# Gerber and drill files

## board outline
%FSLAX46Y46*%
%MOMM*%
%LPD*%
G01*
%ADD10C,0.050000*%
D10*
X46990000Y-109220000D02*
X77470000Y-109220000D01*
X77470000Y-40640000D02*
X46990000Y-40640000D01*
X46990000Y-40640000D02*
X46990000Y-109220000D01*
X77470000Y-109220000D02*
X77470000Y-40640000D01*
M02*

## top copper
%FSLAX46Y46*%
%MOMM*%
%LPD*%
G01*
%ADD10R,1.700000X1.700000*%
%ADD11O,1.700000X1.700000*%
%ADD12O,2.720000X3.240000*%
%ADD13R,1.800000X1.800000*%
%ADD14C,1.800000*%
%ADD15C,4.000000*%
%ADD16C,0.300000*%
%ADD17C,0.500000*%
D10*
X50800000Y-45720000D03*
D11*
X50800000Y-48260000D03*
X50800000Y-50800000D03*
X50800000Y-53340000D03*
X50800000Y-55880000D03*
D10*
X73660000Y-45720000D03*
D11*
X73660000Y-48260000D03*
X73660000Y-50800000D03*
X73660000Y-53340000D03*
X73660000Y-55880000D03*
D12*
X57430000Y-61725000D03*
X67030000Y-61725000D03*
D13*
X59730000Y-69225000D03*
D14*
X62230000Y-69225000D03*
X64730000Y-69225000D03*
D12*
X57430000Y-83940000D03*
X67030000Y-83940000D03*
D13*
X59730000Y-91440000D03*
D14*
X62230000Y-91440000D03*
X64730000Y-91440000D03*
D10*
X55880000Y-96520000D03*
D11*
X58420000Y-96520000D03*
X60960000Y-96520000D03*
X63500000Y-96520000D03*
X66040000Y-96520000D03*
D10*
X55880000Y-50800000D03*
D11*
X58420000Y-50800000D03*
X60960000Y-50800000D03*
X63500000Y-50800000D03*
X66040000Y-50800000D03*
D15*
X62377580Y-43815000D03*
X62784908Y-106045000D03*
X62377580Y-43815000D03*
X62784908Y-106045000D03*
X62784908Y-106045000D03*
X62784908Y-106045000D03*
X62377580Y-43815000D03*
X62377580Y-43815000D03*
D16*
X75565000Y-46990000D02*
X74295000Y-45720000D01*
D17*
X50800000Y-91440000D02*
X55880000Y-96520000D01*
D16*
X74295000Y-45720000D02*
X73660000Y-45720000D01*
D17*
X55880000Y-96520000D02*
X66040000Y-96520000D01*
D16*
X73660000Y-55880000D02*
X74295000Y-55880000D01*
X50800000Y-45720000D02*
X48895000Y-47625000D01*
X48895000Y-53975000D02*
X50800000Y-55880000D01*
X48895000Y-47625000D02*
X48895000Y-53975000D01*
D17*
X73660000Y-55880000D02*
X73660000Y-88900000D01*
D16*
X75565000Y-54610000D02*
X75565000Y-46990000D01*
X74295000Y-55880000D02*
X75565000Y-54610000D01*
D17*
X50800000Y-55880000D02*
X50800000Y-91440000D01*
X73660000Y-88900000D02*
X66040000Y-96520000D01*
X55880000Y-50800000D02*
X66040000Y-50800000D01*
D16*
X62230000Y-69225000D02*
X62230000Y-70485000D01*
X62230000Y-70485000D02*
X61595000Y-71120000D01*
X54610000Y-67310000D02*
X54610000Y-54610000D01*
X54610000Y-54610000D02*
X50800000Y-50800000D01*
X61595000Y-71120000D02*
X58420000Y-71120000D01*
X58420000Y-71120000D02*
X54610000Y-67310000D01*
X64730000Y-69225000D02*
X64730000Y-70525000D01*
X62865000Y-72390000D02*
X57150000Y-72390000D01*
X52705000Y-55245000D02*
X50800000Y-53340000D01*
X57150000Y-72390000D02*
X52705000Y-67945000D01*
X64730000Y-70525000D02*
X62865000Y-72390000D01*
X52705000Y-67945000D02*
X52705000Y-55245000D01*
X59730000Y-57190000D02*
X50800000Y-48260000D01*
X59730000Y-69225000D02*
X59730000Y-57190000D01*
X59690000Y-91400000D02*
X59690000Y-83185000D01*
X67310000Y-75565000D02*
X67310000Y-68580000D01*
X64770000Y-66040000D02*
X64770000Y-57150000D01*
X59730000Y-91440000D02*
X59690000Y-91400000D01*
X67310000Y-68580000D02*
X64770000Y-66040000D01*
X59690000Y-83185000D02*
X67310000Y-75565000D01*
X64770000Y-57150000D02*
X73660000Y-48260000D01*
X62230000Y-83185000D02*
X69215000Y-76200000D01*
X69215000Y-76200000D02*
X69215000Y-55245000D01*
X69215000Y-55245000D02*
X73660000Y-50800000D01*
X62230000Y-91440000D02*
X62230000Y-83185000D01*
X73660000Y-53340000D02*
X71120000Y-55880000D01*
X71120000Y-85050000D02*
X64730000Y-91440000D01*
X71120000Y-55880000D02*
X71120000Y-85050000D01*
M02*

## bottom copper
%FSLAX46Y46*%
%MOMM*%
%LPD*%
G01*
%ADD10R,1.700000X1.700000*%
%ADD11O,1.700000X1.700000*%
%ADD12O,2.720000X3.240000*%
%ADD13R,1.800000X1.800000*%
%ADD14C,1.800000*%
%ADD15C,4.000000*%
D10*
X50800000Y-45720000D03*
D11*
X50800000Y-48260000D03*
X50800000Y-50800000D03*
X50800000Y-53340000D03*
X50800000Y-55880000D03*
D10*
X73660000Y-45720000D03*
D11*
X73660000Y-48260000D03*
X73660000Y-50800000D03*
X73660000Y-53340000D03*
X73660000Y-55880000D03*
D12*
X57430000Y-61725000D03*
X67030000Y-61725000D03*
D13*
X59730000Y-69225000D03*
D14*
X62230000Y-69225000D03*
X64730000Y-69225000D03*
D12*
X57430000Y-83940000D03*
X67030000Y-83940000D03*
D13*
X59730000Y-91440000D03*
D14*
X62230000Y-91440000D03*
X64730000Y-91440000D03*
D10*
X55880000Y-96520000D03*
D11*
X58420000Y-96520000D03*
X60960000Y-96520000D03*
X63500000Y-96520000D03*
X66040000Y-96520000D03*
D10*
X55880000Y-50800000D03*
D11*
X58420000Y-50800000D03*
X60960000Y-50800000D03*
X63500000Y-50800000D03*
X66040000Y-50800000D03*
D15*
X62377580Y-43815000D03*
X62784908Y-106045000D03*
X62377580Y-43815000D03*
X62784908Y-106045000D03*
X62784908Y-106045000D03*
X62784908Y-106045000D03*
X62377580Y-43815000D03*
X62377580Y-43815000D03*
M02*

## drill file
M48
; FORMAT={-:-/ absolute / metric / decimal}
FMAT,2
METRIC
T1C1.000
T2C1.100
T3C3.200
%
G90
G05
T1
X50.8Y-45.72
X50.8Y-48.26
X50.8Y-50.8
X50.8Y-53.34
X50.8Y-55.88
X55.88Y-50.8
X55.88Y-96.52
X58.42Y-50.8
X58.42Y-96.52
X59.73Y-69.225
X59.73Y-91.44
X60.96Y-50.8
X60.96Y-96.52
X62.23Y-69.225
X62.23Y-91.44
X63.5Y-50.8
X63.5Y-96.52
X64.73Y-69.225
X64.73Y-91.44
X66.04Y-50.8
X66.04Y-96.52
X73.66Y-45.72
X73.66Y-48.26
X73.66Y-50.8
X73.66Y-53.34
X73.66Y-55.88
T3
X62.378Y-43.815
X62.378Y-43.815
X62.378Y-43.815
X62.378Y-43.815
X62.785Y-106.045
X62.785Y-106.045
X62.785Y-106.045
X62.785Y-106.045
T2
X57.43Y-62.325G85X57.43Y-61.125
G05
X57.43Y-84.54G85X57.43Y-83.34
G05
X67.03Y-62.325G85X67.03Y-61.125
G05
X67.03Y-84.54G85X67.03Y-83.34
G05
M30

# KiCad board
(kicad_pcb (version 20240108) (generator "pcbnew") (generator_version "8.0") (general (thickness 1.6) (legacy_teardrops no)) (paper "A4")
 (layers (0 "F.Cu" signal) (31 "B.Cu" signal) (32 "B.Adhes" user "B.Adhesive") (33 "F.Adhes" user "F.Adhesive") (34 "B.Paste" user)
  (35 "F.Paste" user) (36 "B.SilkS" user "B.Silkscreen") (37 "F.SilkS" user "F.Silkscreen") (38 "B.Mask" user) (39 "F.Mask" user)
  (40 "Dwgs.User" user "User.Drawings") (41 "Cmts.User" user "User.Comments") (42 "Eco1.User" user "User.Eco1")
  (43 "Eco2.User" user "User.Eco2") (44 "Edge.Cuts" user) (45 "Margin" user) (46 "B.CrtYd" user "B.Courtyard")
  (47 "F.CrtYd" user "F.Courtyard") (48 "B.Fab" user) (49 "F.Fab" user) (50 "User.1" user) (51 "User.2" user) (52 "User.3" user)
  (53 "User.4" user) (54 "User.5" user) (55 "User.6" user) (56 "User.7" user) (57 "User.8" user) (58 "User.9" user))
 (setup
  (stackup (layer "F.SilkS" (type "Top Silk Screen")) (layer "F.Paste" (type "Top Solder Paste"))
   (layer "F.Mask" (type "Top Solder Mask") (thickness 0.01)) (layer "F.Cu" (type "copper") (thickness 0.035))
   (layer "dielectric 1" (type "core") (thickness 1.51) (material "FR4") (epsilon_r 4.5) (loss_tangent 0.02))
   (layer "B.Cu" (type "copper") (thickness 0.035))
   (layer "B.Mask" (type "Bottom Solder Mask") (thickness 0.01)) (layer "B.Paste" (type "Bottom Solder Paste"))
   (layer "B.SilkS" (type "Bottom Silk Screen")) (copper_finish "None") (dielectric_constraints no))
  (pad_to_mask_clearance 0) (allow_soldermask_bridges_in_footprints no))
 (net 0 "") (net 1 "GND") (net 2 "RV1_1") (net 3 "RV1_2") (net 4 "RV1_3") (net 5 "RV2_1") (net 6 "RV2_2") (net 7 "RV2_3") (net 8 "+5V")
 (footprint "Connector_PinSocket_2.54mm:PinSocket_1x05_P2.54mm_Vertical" (layer "F.Cu") (at 50.8 45.72)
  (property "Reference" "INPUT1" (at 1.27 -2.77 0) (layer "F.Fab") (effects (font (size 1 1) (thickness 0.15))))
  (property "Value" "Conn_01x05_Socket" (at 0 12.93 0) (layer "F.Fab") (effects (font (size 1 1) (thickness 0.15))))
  (pad "1" thru_hole rect (at 0 0) (size 1.7 1.7) (drill 1) (layers "*.Cu" "*.Mask") (remove_unused_layers no) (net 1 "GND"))
  (pad "2" thru_hole oval (at 0 2.54) (size 1.7 1.7) (drill 1) (layers "*.Cu" "*.Mask") (remove_unused_layers no) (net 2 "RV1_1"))
  (pad "3" thru_hole oval (at 0 5.08) (size 1.7 1.7) (drill 1) (layers "*.Cu" "*.Mask") (remove_unused_layers no) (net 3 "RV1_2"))
  (pad "4" thru_hole oval (at 0 7.62) (size 1.7 1.7) (drill 1) (layers "*.Cu" "*.Mask") (remove_unused_layers no) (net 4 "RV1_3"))
  (pad "5" thru_hole oval (at 0 10.16) (size 1.7 1.7) (drill 1) (layers "*.Cu" "*.Mask") (remove_unused_layers no) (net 1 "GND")))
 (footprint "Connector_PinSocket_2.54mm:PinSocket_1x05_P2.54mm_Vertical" (layer "F.Cu") (at 73.66 45.72)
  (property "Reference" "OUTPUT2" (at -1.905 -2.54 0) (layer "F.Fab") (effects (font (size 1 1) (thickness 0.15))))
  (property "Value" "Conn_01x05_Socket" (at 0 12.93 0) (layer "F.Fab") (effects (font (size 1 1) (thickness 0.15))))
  (pad "1" thru_hole rect (at 0 0) (size 1.7 1.7) (drill 1) (layers "*.Cu" "*.Mask") (remove_unused_layers no) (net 1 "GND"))
  (pad "2" thru_hole oval (at 0 2.54) (size 1.7 1.7) (drill 1) (layers "*.Cu" "*.Mask") (remove_unused_layers no) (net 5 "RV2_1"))
  (pad "3" thru_hole oval (at 0 5.08) (size 1.7 1.7) (drill 1) (layers "*.Cu" "*.Mask") (remove_unused_layers no) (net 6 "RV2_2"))
  (pad "4" thru_hole oval (at 0 7.62) (size 1.7 1.7) (drill 1) (layers "*.Cu" "*.Mask") (remove_unused_layers no) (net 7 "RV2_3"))
  (pad "5" thru_hole oval (at 0 10.16) (size 1.7 1.7) (drill 1) (layers "*.Cu" "*.Mask") (remove_unused_layers no) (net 1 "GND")))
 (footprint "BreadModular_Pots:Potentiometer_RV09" (layer "F.Cu") (at 59.73 69.225 90)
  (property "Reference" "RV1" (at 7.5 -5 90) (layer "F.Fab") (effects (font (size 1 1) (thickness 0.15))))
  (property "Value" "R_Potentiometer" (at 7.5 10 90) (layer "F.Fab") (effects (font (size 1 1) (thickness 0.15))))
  (pad "" thru_hole oval (at 7.5 -2.3 180) (size 2.72 3.24) (drill oval 1.1 2.3) (layers "*.Cu" "*.Mask") (remove_unused_layers no))
  (pad "" thru_hole oval (at 7.5 7.3 180) (size 2.72 3.24) (drill oval 1.1 2.3) (layers "*.Cu" "*.Mask") (remove_unused_layers no))
  (pad "1" thru_hole rect (at 0 0 180) (size 1.8 1.8) (drill 1) (layers "*.Cu" "*.Mask") (remove_unused_layers no) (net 2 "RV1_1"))
  (pad "2" thru_hole circle (at 0 2.5 180) (size 1.8 1.8) (drill 1) (layers "*.Cu" "*.Mask") (remove_unused_layers no) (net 3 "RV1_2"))
  (pad "3" thru_hole circle (at 0 5 180) (size 1.8 1.8) (drill 1) (layers "*.Cu" "*.Mask") (remove_unused_layers no) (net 4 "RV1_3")))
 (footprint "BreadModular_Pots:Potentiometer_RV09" (layer "F.Cu") (at 59.73 91.44 90)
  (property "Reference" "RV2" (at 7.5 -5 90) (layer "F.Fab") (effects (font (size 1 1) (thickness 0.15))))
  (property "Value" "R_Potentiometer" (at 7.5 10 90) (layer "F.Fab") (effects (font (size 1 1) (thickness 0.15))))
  (pad "" thru_hole oval (at 7.5 -2.3 180) (size 2.72 3.24) (drill oval 1.1 2.3) (layers "*.Cu" "*.Mask") (remove_unused_layers no))
  (pad "" thru_hole oval (at 7.5 7.3 180) (size 2.72 3.24) (drill oval 1.1 2.3) (layers "*.Cu" "*.Mask") (remove_unused_layers no))
  (pad "1" thru_hole rect (at 0 0 180) (size 1.8 1.8) (drill 1) (layers "*.Cu" "*.Mask") (remove_unused_layers no) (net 5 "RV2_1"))
  (pad "2" thru_hole circle (at 0 2.5 180) (size 1.8 1.8) (drill 1) (layers "*.Cu" "*.Mask") (remove_unused_layers no) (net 6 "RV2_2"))
  (pad "3" thru_hole circle (at 0 5 180) (size 1.8 1.8) (drill 1) (layers "*.Cu" "*.Mask") (remove_unused_layers no) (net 7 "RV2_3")))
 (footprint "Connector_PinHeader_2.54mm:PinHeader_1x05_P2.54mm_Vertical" (layer "B.Cu") (at 55.88 96.52 -90)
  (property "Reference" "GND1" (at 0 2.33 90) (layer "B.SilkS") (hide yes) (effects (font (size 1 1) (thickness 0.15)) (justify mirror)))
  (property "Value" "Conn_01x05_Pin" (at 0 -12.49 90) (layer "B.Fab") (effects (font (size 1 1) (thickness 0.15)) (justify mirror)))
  (pad "1" thru_hole rect (at 0 0 270) (size 1.7 1.7) (drill 1) (layers "*.Cu" "*.Mask") (remove_unused_layers no) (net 1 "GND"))
  (pad "2" thru_hole oval (at 0 -2.54 270) (size 1.7 1.7) (drill 1) (layers "*.Cu" "*.Mask") (remove_unused_layers no) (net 1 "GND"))
  (pad "3" thru_hole oval (at 0 -5.08 270) (size 1.7 1.7) (drill 1) (layers "*.Cu" "*.Mask") (remove_unused_layers no) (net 1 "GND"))
  (pad "4" thru_hole oval (at 0 -7.62 270) (size 1.7 1.7) (drill 1) (layers "*.Cu" "*.Mask") (remove_unused_layers no) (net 1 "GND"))
  (pad "5" thru_hole oval (at 0 -10.16 270) (size 1.7 1.7) (drill 1) (layers "*.Cu" "*.Mask") (remove_unused_layers no) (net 1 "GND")))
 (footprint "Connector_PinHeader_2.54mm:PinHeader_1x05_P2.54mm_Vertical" (layer "B.Cu") (at 55.88 50.8 -90)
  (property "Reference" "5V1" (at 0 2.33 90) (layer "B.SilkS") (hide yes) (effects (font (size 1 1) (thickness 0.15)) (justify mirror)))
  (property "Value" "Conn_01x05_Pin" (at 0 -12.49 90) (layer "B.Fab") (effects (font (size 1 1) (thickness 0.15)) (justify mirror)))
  (pad "1" thru_hole rect (at 0 0 270) (size 1.7 1.7) (drill 1) (layers "*.Cu" "*.Mask") (remove_unused_layers no) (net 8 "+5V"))
  (pad "2" thru_hole oval (at 0 -2.54 270) (size 1.7 1.7) (drill 1) (layers "*.Cu" "*.Mask") (remove_unused_layers no) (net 8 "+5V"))
  (pad "3" thru_hole oval (at 0 -5.08 270) (size 1.7 1.7) (drill 1) (layers "*.Cu" "*.Mask") (remove_unused_layers no) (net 8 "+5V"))
  (pad "4" thru_hole oval (at 0 -7.62 270) (size 1.7 1.7) (drill 1) (layers "*.Cu" "*.Mask") (remove_unused_layers no) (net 8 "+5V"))
  (pad "5" thru_hole oval (at 0 -10.16 270) (size 1.7 1.7) (drill 1) (layers "*.Cu" "*.Mask") (remove_unused_layers no) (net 8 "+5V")))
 (gr_line (start 46.99 109.22) (end 77.47 109.22) (stroke (width 0.05) (type default)) (layer "Edge.Cuts"))
 (gr_line (start 77.47 40.64) (end 46.99 40.64) (stroke (width 0.05) (type default)) (layer "Edge.Cuts"))
 (gr_line (start 46.99 40.64) (end 46.99 109.22) (stroke (width 0.05) (type default)) (layer "Edge.Cuts"))
 (gr_line (start 77.47 109.22) (end 77.47 40.64) (stroke (width 0.05) (type default)) (layer "Edge.Cuts"))
 (via (at 62.37758 43.815) (size 4) (drill 3.2) (layers "F.Cu" "B.Cu") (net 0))
 (via (at 62.784908 106.045) (size 4) (drill 3.2) (layers "F.Cu" "B.Cu") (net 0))
 (via (at 62.37758 43.815) (size 4) (drill 3.2) (layers "F.Cu" "B.Cu") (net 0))
 (via (at 62.784908 106.045) (size 4) (drill 3.2) (layers "F.Cu" "B.Cu") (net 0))
 (via (at 62.784908 106.045) (size 4) (drill 3.2) (layers "F.Cu" "B.Cu") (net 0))
 (via (at 62.784908 106.045) (size 4) (drill 3.2) (layers "F.Cu" "B.Cu") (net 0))
 (via (at 62.37758 43.815) (size 4) (drill 3.2) (layers "F.Cu" "B.Cu") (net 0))
 (via (at 62.37758 43.815) (size 4) (drill 3.2) (layers "F.Cu" "B.Cu") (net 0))
 (segment (start 75.565 46.99) (end 74.295 45.72) (width 0.3) (layer "F.Cu") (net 1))
 (segment (start 50.8 91.44) (end 55.88 96.52) (width 0.5) (layer "F.Cu") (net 1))
 (segment (start 74.295 45.72) (end 73.66 45.72) (width 0.3) (layer "F.Cu") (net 1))
 (segment (start 55.88 96.52) (end 66.04 96.52) (width 0.5) (layer "F.Cu") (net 1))
 (segment (start 73.66 55.88) (end 74.295 55.88) (width 0.3) (layer "F.Cu") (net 1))
 (segment (start 50.8 45.72) (end 48.895 47.625) (width 0.3) (layer "F.Cu") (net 1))
 (segment (start 48.895 53.975) (end 50.8 55.88) (width 0.3) (layer "F.Cu") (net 1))
 (segment (start 48.895 47.625) (end 48.895 53.975) (width 0.3) (layer "F.Cu") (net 1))
 (segment (start 73.66 55.88) (end 73.66 88.9) (width 0.5) (layer "F.Cu") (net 1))
 (segment (start 75.565 54.61) (end 75.565 46.99) (width 0.3) (layer "F.Cu") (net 1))
 (segment (start 74.295 55.88) (end 75.565 54.61) (width 0.3) (layer "F.Cu") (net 1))
 (segment (start 50.8 55.88) (end 50.8 91.44) (width 0.5) (layer "F.Cu") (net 1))
 (segment (start 73.66 88.9) (end 66.04 96.52) (width 0.5) (layer "F.Cu") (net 1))
 (segment (start 55.88 50.8) (end 66.04 50.8) (width 0.5) (layer "F.Cu") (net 8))
 (segment (start 62.23 69.225) (end 62.23 70.485) (width 0.3) (layer "F.Cu") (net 3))
 (segment (start 62.23 70.485) (end 61.595 71.12) (width 0.3) (layer "F.Cu") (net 3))
 (segment (start 54.61 67.31) (end 54.61 54.61) (width 0.3) (layer "F.Cu") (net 3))
 (segment (start 54.61 54.61) (end 50.8 50.8) (width 0.3) (layer "F.Cu") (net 3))
 (segment (start 61.595 71.12) (end 58.42 71.12) (width 0.3) (layer "F.Cu") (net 3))
 (segment (start 58.42 71.12) (end 54.61 67.31) (width 0.3) (layer "F.Cu") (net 3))
 (segment (start 64.73 69.225) (end 64.73 70.525) (width 0.3) (layer "F.Cu") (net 4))
 (segment (start 62.865 72.39) (end 57.15 72.39) (width 0.3) (layer "F.Cu") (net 4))
 (segment (start 52.705 55.245) (end 50.8 53.34) (width 0.3) (layer "F.Cu") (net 4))
 (segment (start 57.15 72.39) (end 52.705 67.945) (width 0.3) (layer "F.Cu") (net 4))
 (segment (start 64.73 70.525) (end 62.865 72.39) (width 0.3) (layer "F.Cu") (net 4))
 (segment (start 52.705 67.945) (end 52.705 55.245) (width 0.3) (layer "F.Cu") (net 4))
 (segment (start 59.73 57.19) (end 50.8 48.26) (width 0.3) (layer "F.Cu") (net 2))
 (segment (start 59.73 69.225) (end 59.73 57.19) (width 0.3) (layer "F.Cu") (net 2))
 (segment (start 59.69 91.4) (end 59.69 83.185) (width 0.3) (layer "F.Cu") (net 5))
 (segment (start 67.31 75.565) (end 67.31 68.58) (width 0.3) (layer "F.Cu") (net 5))
 (segment (start 64.77 66.04) (end 64.77 57.15) (width 0.3) (layer "F.Cu") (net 5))
 (segment (start 59.73 91.44) (end 59.69 91.4) (width 0.3) (layer "F.Cu") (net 5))
 (segment (start 67.31 68.58) (end 64.77 66.04) (width 0.3) (layer "F.Cu") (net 5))
 (segment (start 59.69 83.185) (end 67.31 75.565) (width 0.3) (layer "F.Cu") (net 5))
 (segment (start 64.77 57.15) (end 73.66 48.26) (width 0.3) (layer "F.Cu") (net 5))
 (segment (start 62.23 83.185) (end 69.215 76.2) (width 0.3) (layer "F.Cu") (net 6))
 (segment (start 69.215 76.2) (end 69.215 55.245) (width 0.3) (layer "F.Cu") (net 6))
 (segment (start 69.215 55.245) (end 73.66 50.8) (width 0.3) (layer "F.Cu") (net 6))
 (segment (start 62.23 91.44) (end 62.23 83.185) (width 0.3) (layer "F.Cu") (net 6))
 (segment (start 73.66 53.34) (end 71.12 55.88) (width 0.3) (layer "F.Cu") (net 7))
 (segment (start 71.12 85.05) (end 64.73 91.44) (width 0.3) (layer "F.Cu") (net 7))
 (segment (start 71.12 55.88) (end 71.12 85.05) (width 0.3) (layer "F.Cu") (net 7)))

